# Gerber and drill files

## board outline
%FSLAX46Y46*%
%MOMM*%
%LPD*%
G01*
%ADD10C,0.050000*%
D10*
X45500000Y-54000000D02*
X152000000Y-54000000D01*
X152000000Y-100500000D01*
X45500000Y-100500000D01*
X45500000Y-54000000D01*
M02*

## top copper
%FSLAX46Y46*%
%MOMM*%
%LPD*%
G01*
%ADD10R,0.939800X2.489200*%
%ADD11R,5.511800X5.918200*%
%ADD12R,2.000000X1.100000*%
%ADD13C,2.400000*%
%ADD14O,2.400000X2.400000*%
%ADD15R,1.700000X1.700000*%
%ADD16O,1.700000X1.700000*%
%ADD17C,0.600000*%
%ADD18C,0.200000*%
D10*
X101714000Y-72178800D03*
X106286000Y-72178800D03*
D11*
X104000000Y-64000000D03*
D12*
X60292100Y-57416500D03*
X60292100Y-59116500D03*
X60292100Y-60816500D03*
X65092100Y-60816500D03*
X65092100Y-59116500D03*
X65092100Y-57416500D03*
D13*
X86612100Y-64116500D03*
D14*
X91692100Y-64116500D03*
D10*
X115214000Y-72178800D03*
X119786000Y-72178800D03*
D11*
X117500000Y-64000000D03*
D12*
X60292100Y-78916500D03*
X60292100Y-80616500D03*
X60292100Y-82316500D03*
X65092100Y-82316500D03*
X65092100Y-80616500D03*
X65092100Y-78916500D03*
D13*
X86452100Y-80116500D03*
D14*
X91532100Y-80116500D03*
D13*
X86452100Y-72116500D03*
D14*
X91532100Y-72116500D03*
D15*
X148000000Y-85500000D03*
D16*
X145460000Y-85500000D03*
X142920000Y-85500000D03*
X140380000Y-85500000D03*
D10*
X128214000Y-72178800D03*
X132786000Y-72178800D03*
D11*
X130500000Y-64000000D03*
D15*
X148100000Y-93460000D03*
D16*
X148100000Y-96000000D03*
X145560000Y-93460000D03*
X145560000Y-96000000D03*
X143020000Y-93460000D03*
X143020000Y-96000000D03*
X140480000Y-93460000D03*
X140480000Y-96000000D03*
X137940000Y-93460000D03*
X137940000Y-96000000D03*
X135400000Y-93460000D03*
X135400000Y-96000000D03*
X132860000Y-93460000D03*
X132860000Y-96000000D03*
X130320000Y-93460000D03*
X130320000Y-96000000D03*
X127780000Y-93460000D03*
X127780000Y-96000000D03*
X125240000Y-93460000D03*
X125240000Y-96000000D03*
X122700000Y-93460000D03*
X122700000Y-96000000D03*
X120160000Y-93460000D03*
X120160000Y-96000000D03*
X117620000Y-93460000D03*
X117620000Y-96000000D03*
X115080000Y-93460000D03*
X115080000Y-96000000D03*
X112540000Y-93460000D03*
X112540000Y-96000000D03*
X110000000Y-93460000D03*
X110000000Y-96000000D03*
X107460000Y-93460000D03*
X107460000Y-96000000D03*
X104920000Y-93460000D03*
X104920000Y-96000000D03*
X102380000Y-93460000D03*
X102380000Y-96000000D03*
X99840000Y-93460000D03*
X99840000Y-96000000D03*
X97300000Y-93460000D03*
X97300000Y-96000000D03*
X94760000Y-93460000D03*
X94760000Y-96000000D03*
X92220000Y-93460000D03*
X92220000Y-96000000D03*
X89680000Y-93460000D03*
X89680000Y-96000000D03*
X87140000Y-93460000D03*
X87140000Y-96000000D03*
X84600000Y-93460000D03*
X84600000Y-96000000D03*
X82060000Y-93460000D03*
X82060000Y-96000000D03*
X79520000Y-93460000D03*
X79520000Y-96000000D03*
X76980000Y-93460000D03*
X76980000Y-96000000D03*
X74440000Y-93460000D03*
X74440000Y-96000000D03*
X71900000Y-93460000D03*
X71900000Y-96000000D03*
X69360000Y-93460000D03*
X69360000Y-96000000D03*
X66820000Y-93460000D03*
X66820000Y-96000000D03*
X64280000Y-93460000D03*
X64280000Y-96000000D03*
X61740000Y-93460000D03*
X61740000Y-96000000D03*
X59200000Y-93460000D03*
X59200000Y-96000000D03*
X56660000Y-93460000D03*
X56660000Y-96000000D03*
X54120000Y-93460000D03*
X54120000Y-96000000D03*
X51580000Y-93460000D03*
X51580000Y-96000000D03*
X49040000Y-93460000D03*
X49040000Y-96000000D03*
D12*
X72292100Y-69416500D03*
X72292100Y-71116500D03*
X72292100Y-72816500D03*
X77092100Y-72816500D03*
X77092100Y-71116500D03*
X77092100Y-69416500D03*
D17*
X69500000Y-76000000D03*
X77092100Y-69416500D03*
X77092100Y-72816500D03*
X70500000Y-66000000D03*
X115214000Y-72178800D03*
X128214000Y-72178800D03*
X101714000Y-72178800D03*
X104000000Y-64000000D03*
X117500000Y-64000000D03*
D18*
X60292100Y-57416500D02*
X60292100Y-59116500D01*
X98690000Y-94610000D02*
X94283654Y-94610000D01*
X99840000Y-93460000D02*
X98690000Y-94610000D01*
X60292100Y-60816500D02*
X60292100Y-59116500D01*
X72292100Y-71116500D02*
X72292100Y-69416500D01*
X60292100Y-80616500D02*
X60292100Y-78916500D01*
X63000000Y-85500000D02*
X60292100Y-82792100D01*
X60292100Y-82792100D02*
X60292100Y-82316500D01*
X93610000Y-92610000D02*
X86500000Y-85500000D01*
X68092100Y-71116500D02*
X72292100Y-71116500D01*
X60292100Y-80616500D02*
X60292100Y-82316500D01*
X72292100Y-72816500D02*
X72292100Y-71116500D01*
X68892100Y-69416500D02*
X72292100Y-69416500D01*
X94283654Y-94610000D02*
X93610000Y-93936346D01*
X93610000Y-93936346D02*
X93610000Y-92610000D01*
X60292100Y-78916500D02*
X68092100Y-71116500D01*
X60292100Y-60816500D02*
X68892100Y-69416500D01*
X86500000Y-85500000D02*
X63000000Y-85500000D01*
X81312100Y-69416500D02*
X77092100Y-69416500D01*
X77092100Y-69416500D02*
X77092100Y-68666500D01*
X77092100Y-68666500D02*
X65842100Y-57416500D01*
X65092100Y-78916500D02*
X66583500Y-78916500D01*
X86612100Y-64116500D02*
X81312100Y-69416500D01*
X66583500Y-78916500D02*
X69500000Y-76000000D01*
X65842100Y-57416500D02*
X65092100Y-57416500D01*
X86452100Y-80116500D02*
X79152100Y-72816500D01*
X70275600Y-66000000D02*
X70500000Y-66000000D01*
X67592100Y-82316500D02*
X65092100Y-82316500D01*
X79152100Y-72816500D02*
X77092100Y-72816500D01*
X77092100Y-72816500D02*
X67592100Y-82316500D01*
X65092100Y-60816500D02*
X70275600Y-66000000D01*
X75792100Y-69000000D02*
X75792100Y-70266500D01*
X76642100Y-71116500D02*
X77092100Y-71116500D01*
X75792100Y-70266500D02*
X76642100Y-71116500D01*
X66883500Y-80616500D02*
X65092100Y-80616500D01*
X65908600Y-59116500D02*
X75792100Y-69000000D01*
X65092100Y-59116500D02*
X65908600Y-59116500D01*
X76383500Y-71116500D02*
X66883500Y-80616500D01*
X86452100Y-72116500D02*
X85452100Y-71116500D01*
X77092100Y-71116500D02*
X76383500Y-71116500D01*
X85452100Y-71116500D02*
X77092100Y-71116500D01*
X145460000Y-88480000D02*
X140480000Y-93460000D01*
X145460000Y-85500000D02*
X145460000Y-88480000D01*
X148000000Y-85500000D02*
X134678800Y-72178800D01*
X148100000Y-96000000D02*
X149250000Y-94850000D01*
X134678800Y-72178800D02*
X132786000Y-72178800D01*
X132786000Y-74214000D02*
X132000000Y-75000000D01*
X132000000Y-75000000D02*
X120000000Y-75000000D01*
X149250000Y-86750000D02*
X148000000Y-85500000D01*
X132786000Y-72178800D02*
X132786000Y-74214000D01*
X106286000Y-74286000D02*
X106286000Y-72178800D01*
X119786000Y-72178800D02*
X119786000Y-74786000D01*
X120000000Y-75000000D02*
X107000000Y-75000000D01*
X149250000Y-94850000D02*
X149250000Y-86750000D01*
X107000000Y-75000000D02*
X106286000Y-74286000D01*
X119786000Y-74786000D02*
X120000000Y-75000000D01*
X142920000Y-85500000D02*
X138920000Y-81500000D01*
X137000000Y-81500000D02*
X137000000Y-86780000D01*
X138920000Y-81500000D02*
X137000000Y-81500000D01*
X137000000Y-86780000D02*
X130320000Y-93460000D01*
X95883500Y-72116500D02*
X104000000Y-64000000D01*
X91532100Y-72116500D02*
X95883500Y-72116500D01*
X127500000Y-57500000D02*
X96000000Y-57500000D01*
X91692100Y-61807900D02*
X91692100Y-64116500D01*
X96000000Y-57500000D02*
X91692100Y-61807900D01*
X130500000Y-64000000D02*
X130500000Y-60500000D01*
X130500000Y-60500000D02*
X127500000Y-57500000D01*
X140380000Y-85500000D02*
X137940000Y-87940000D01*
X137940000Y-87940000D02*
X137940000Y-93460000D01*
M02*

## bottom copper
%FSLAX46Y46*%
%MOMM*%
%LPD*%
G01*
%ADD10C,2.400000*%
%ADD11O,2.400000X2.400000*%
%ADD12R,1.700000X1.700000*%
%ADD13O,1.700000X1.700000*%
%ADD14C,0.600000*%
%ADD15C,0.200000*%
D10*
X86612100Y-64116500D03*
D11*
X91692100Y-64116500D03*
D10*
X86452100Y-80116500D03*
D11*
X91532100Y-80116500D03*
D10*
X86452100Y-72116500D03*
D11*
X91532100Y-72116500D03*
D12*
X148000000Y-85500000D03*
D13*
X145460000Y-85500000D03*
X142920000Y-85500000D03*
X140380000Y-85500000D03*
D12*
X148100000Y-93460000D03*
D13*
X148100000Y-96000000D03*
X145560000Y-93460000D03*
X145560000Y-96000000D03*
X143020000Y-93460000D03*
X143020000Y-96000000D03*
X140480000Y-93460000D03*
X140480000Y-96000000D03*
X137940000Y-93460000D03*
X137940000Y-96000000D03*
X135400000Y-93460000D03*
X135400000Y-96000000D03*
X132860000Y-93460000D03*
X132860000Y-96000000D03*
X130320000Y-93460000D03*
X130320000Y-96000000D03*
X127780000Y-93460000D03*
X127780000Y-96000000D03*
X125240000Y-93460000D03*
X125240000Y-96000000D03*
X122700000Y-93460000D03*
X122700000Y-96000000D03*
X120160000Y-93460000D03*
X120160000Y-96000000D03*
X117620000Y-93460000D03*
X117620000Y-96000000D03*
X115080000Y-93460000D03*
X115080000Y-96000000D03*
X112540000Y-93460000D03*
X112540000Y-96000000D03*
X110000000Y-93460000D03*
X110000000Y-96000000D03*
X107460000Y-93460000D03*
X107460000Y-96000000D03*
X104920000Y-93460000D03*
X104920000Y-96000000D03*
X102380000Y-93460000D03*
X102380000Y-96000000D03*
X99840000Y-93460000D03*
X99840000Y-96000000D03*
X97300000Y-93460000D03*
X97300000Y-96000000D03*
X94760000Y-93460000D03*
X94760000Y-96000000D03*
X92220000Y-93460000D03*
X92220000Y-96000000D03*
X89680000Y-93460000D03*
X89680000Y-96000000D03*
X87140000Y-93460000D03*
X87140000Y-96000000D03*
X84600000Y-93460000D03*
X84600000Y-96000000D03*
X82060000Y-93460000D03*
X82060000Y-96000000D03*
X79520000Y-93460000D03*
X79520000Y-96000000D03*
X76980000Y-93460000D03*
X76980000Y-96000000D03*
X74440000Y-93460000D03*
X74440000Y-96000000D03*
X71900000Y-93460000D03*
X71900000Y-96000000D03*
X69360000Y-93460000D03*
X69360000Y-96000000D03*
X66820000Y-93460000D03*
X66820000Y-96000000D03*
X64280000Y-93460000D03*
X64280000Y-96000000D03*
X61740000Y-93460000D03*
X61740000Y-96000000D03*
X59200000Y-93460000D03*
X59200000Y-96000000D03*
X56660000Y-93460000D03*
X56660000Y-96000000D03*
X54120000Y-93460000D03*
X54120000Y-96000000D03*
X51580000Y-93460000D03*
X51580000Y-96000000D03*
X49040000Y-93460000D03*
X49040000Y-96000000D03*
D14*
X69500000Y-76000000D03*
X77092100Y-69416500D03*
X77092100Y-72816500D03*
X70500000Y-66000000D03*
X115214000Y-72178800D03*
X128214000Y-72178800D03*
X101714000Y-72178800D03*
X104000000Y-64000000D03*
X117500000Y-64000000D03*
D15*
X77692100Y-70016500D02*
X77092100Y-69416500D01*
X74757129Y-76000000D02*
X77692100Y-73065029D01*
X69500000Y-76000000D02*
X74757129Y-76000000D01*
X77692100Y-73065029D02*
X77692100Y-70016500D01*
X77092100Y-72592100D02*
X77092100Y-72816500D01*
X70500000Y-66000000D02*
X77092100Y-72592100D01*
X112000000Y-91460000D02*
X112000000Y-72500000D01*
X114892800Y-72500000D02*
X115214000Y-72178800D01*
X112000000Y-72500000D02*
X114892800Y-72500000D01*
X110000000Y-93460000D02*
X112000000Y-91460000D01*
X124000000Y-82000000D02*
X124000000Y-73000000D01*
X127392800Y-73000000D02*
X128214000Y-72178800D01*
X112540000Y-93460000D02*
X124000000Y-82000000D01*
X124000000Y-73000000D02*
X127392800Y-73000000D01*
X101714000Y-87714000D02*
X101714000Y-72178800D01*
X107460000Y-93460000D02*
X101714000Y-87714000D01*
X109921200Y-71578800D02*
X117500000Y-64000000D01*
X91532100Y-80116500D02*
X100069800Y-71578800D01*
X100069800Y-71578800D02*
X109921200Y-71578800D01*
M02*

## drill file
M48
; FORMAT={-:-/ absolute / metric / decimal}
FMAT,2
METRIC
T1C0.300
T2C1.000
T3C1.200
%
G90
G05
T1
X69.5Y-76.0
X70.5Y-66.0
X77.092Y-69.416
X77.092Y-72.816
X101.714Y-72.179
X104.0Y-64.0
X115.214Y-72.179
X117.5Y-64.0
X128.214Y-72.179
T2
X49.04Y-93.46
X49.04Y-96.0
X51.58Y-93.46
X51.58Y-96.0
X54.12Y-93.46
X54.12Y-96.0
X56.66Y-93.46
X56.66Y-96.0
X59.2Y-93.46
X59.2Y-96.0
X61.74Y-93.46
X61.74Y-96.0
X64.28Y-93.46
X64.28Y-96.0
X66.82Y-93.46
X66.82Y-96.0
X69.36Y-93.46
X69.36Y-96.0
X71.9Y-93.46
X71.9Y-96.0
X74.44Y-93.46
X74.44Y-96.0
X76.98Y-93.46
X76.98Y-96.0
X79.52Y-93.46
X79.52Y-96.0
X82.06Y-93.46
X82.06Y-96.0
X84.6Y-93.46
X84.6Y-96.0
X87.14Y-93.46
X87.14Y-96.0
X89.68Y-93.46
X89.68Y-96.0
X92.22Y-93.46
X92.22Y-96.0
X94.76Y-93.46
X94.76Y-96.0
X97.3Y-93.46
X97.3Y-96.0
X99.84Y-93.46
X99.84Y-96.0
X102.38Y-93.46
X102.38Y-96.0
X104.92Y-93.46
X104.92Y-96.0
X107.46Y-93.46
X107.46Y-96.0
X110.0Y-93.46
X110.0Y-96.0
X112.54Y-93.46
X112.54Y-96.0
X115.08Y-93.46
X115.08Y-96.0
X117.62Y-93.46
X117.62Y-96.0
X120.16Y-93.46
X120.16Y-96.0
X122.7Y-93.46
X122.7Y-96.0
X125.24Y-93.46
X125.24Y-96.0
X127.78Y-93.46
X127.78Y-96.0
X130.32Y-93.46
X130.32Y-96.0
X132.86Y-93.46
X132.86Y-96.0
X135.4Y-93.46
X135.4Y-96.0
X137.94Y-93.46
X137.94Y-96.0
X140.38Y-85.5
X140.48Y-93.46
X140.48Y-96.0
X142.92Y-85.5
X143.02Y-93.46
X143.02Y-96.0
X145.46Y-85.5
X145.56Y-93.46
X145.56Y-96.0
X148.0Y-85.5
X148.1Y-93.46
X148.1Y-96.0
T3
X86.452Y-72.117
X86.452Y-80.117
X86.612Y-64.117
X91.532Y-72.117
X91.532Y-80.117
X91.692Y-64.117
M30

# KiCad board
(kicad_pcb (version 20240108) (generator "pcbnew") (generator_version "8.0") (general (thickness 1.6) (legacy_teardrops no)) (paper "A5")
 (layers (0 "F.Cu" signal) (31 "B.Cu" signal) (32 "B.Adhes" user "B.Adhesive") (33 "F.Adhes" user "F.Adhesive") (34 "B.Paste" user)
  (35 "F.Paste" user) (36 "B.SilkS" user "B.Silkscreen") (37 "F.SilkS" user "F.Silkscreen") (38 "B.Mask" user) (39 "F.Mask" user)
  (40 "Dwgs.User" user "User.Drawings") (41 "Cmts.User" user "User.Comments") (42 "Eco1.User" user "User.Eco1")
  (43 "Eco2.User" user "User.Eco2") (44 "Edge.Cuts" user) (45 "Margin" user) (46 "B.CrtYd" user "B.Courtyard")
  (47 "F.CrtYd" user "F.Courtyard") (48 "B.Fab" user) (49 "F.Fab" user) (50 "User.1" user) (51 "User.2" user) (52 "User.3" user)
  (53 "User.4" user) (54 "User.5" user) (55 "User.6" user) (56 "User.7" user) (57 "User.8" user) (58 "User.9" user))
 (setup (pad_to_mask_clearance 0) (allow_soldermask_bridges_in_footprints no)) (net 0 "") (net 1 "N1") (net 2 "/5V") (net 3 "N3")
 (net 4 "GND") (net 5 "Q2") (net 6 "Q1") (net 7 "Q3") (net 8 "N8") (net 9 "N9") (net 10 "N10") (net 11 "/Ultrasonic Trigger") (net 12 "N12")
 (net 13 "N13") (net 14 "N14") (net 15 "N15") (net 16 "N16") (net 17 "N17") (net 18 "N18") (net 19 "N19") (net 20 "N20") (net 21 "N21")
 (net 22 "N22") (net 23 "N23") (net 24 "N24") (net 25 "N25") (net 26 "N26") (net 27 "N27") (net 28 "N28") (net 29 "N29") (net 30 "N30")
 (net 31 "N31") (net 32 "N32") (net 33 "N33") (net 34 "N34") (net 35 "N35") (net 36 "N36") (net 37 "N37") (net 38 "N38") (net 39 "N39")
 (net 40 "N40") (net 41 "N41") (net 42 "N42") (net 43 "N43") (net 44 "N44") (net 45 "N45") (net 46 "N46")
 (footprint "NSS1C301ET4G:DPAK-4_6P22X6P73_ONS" (layer "F.Cu") (at 104 65.7653)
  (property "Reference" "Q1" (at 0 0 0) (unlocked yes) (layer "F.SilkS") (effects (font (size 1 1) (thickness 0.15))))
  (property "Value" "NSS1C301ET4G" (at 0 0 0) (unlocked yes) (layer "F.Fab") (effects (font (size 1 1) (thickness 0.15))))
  (pad "1" smd rect (at -2.286 6.4135) (size 0.9398 2.4892) (layers "F.Cu" "F.Paste" "F.Mask") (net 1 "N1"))
  (pad "2" smd rect (at 2.286 6.4135) (size 0.9398 2.4892) (layers "F.Cu" "F.Paste" "F.Mask") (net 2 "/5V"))
  (pad "3" smd rect (at 0 -1.7653) (size 5.5118 5.9182) (layers "F.Cu" "F.Paste" "F.Mask") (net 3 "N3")))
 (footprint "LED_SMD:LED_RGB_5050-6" (layer "F.Cu") (at 62.6921 59.1165)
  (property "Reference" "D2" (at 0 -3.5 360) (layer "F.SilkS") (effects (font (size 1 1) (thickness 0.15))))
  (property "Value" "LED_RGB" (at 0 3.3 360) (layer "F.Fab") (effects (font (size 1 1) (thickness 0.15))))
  (pad "1" smd rect (at -2.4 -1.7 90) (size 1.1 2) (layers "F.Cu" "F.Paste" "F.Mask") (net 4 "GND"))
  (pad "2" smd rect (at -2.4 0 90) (size 1.1 2) (layers "F.Cu" "F.Paste" "F.Mask") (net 4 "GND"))
  (pad "3" smd rect (at -2.4 1.7 90) (size 1.1 2) (layers "F.Cu" "F.Paste" "F.Mask") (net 4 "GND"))
  (pad "4" smd rect (at 2.4 1.7 90) (size 1.1 2) (layers "F.Cu" "F.Paste" "F.Mask") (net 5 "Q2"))
  (pad "5" smd rect (at 2.4 0 90) (size 1.1 2) (layers "F.Cu" "F.Paste" "F.Mask") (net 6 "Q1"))
  (pad "6" smd rect (at 2.4 -1.7 90) (size 1.1 2) (layers "F.Cu" "F.Paste" "F.Mask") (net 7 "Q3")))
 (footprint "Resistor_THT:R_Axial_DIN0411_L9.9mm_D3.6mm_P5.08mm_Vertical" (layer "F.Cu") (at 86.6121 64.1165)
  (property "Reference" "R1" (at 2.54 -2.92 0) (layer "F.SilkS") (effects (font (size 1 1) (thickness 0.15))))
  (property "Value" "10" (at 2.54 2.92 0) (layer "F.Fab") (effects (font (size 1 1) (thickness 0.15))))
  (pad "1" thru_hole circle (at 0 0) (size 2.4 2.4) (drill 1.2) (layers "*.Cu" "*.Mask") (remove_unused_layers no) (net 7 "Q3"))
  (pad "2" thru_hole oval (at 5.08 0) (size 2.4 2.4) (drill 1.2) (layers "*.Cu" "*.Mask") (remove_unused_layers no) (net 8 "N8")))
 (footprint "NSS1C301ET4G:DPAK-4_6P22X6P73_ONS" (layer "F.Cu") (at 117.5 65.7653)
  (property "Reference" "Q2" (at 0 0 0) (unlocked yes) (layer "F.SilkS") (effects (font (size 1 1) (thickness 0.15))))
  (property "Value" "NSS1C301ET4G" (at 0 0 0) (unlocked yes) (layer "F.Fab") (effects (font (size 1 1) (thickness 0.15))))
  (pad "1" smd rect (at -2.286 6.4135) (size 0.9398 2.4892) (layers "F.Cu" "F.Paste" "F.Mask") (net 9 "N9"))
  (pad "2" smd rect (at 2.286 6.4135) (size 0.9398 2.4892) (layers "F.Cu" "F.Paste" "F.Mask") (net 2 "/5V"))
  (pad "3" smd rect (at 0 -1.7653) (size 5.5118 5.9182) (layers "F.Cu" "F.Paste" "F.Mask") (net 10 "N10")))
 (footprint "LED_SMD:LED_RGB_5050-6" (layer "F.Cu") (at 62.6921 80.6165)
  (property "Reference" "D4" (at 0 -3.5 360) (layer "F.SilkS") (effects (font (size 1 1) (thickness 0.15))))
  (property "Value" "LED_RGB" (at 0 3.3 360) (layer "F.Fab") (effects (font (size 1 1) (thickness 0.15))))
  (pad "1" smd rect (at -2.4 -1.7 90) (size 1.1 2) (layers "F.Cu" "F.Paste" "F.Mask") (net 4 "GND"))
  (pad "2" smd rect (at -2.4 0 90) (size 1.1 2) (layers "F.Cu" "F.Paste" "F.Mask") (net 4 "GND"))
  (pad "3" smd rect (at -2.4 1.7 90) (size 1.1 2) (layers "F.Cu" "F.Paste" "F.Mask") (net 4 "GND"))
  (pad "4" smd rect (at 2.4 1.7 90) (size 1.1 2) (layers "F.Cu" "F.Paste" "F.Mask") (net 5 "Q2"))
  (pad "5" smd rect (at 2.4 0 90) (size 1.1 2) (layers "F.Cu" "F.Paste" "F.Mask") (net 6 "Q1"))
  (pad "6" smd rect (at 2.4 -1.7 90) (size 1.1 2) (layers "F.Cu" "F.Paste" "F.Mask") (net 7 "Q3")))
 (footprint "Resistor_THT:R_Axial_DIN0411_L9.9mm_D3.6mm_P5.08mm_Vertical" (layer "F.Cu") (at 86.4521 80.1165)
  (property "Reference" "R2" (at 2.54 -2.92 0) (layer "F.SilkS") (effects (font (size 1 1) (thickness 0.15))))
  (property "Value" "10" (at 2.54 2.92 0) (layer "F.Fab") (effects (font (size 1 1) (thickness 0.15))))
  (pad "1" thru_hole circle (at 0 0) (size 2.4 2.4) (drill 1.2) (layers "*.Cu" "*.Mask") (remove_unused_layers no) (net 5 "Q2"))
  (pad "2" thru_hole oval (at 5.08 0) (size 2.4 2.4) (drill 1.2) (layers "*.Cu" "*.Mask") (remove_unused_layers no) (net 10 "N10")))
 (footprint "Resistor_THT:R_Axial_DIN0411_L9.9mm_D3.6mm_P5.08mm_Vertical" (layer "F.Cu") (at 86.4521 72.1165)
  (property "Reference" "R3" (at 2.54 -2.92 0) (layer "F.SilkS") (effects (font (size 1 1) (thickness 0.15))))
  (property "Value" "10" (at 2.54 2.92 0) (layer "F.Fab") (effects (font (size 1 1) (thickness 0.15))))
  (pad "1" thru_hole circle (at 0 0) (size 2.4 2.4) (drill 1.2) (layers "*.Cu" "*.Mask") (remove_unused_layers no) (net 6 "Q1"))
  (pad "2" thru_hole oval (at 5.08 0) (size 2.4 2.4) (drill 1.2) (layers "*.Cu" "*.Mask") (remove_unused_layers no) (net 3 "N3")))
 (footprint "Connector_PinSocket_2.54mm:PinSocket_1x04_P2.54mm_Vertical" (layer "F.Cu") (at 148 85.5 -90)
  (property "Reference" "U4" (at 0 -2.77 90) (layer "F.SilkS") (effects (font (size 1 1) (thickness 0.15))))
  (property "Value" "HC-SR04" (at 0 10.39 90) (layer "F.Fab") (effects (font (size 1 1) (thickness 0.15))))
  (pad "1" thru_hole rect (at 0 0 270) (size 1.7 1.7) (drill 1) (layers "*.Cu" "*.Mask") (remove_unused_layers no) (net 2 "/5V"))
  (pad "2" thru_hole oval (at 0 2.54 270) (size 1.7 1.7) (drill 1) (layers "*.Cu" "*.Mask") (remove_unused_layers no)
   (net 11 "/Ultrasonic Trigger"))
  (pad "3" thru_hole oval (at 0 5.08 270) (size 1.7 1.7) (drill 1) (layers "*.Cu" "*.Mask") (remove_unused_layers no) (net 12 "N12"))
  (pad "4" thru_hole oval (at 0 7.62 270) (size 1.7 1.7) (drill 1) (layers "*.Cu" "*.Mask") (remove_unused_layers no) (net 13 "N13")))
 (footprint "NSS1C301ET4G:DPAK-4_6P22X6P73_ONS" (layer "F.Cu") (at 130.5 65.7653)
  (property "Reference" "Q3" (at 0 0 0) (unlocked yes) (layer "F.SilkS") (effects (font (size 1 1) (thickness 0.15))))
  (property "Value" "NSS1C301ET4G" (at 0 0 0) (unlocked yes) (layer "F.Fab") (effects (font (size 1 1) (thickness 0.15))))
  (pad "1" smd rect (at -2.286 6.4135) (size 0.9398 2.4892) (layers "F.Cu" "F.Paste" "F.Mask") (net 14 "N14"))
  (pad "2" smd rect (at 2.286 6.4135) (size 0.9398 2.4892) (layers "F.Cu" "F.Paste" "F.Mask") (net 2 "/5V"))
  (pad "3" smd rect (at 0 -1.7653) (size 5.5118 5.9182) (layers "F.Cu" "F.Paste" "F.Mask") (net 8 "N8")))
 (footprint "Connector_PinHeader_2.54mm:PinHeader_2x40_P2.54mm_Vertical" (layer "F.Cu") (at 148.1 93.46 -90)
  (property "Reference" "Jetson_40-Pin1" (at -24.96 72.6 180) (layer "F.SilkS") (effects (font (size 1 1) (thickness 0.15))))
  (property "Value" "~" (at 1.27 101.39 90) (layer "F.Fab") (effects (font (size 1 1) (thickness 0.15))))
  (pad "1" thru_hole rect (at 0 0 270) (size 1.7 1.7) (drill 1) (layers "*.Cu" "*.Mask") (remove_unused_layers no) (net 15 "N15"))
  (pad "2" thru_hole oval (at 2.54 0 270) (size 1.7 1.7) (drill 1) (layers "*.Cu" "*.Mask") (remove_unused_layers no) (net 2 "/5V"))
  (pad "3" thru_hole oval (at 0 2.54 270) (size 1.7 1.7) (drill 1) (layers "*.Cu" "*.Mask") (remove_unused_layers no) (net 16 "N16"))
  (pad "4" thru_hole oval (at 2.54 2.54 270) (size 1.7 1.7) (drill 1) (layers "*.Cu" "*.Mask") (remove_unused_layers no) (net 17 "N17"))
  (pad "5" thru_hole oval (at 0 5.08 270) (size 1.7 1.7) (drill 1) (layers "*.Cu" "*.Mask") (remove_unused_layers no) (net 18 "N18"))
  (pad "6" thru_hole oval (at 2.54 5.08 270) (size 1.7 1.7) (drill 1) (layers "*.Cu" "*.Mask") (remove_unused_layers no) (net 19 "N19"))
  (pad "7" thru_hole oval (at 0 7.62 270) (size 1.7 1.7) (drill 1) (layers "*.Cu" "*.Mask") (remove_unused_layers no)
   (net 11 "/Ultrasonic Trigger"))
  (pad "8" thru_hole oval (at 2.54 7.62 270) (size 1.7 1.7) (drill 1) (layers "*.Cu" "*.Mask") (remove_unused_layers no) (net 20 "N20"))
  (pad "9" thru_hole oval (at 0 10.16 270) (size 1.7 1.7) (drill 1) (layers "*.Cu" "*.Mask") (remove_unused_layers no) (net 13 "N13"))
  (pad "10" thru_hole oval (at 2.54 10.16 270) (size 1.7 1.7) (drill 1) (layers "*.Cu" "*.Mask") (remove_unused_layers no) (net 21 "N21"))
  (pad "11" thru_hole oval (at 0 12.7 270) (size 1.7 1.7) (drill 1) (layers "*.Cu" "*.Mask") (remove_unused_layers no) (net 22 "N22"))
  (pad "12" thru_hole oval (at 2.54 12.7 270) (size 1.7 1.7) (drill 1) (layers "*.Cu" "*.Mask") (remove_unused_layers no) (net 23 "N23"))
  (pad "13" thru_hole oval (at 0 15.24 270) (size 1.7 1.7) (drill 1) (layers "*.Cu" "*.Mask") (remove_unused_layers no) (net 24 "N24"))
  (pad "14" thru_hole oval (at 2.54 15.24 270) (size 1.7 1.7) (drill 1) (layers "*.Cu" "*.Mask") (remove_unused_layers no) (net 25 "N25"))
  (pad "15" thru_hole oval (at 0 17.78 270) (size 1.7 1.7) (drill 1) (layers "*.Cu" "*.Mask") (remove_unused_layers no) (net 12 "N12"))
  (pad "16" thru_hole oval (at 2.54 17.78 270) (size 1.7 1.7) (drill 1) (layers "*.Cu" "*.Mask") (remove_unused_layers no) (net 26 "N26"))
  (pad "17" thru_hole oval (at 0 20.32 270) (size 1.7 1.7) (drill 1) (layers "*.Cu" "*.Mask") (remove_unused_layers no) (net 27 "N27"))
  (pad "18" thru_hole oval (at 2.54 20.32 270) (size 1.7 1.7) (drill 1) (layers "*.Cu" "*.Mask") (remove_unused_layers no) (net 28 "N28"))
  (pad "19" thru_hole oval (at 0 22.86 270) (size 1.7 1.7) (drill 1) (layers "*.Cu" "*.Mask") (remove_unused_layers no) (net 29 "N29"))
  (pad "20" thru_hole oval (at 2.54 22.86 270) (size 1.7 1.7) (drill 1) (layers "*.Cu" "*.Mask") (remove_unused_layers no) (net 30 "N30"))
  (pad "21" thru_hole oval (at 0 25.4 270) (size 1.7 1.7) (drill 1) (layers "*.Cu" "*.Mask") (remove_unused_layers no) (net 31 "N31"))
  (pad "22" thru_hole oval (at 2.54 25.4 270) (size 1.7 1.7) (drill 1) (layers "*.Cu" "*.Mask") (remove_unused_layers no) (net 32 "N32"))
  (pad "23" thru_hole oval (at 0 27.94 270) (size 1.7 1.7) (drill 1) (layers "*.Cu" "*.Mask") (remove_unused_layers no) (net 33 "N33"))
  (pad "24" thru_hole oval (at 2.54 27.94 270) (size 1.7 1.7) (drill 1) (layers "*.Cu" "*.Mask") (remove_unused_layers no) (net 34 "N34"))
  (pad "25" thru_hole oval (at 0 30.48 270) (size 1.7 1.7) (drill 1) (layers "*.Cu" "*.Mask") (remove_unused_layers no) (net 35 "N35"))
  (pad "26" thru_hole oval (at 2.54 30.48 270) (size 1.7 1.7) (drill 1) (layers "*.Cu" "*.Mask") (remove_unused_layers no) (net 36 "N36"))
  (pad "27" thru_hole oval (at 0 33.02 270) (size 1.7 1.7) (drill 1) (layers "*.Cu" "*.Mask") (remove_unused_layers no) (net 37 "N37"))
  (pad "28" thru_hole oval (at 2.54 33.02 270) (size 1.7 1.7) (drill 1) (layers "*.Cu" "*.Mask") (remove_unused_layers no) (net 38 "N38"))
  (pad "29" thru_hole oval (at 0 35.56 270) (size 1.7 1.7) (drill 1) (layers "*.Cu" "*.Mask") (remove_unused_layers no) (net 14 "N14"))
  (pad "30" thru_hole oval (at 2.54 35.56 270) (size 1.7 1.7) (drill 1) (layers "*.Cu" "*.Mask") (remove_unused_layers no) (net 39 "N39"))
  (pad "31" thru_hole oval (at 0 38.1 270) (size 1.7 1.7) (drill 1) (layers "*.Cu" "*.Mask") (remove_unused_layers no) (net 9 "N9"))
  (pad "32" thru_hole oval (at 2.54 38.1 270) (size 1.7 1.7) (drill 1) (layers "*.Cu" "*.Mask") (remove_unused_layers no) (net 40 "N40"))
  (pad "33" thru_hole oval (at 0 40.64 270) (size 1.7 1.7) (drill 1) (layers "*.Cu" "*.Mask") (remove_unused_layers no) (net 1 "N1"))
  (pad "34" thru_hole oval (at 2.54 40.64 270) (size 1.7 1.7) (drill 1) (layers "*.Cu" "*.Mask") (remove_unused_layers no) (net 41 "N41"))
  (pad "35" thru_hole oval (at 0 43.18 270) (size 1.7 1.7) (drill 1) (layers "*.Cu" "*.Mask") (remove_unused_layers no) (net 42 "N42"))
  (pad "36" thru_hole oval (at 2.54 43.18 270) (size 1.7 1.7) (drill 1) (layers "*.Cu" "*.Mask") (remove_unused_layers no) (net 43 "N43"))
  (pad "37" thru_hole oval (at 0 45.72 270) (size 1.7 1.7) (drill 1) (layers "*.Cu" "*.Mask") (remove_unused_layers no) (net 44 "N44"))
  (pad "38" thru_hole oval (at 2.54 45.72 270) (size 1.7 1.7) (drill 1) (layers "*.Cu" "*.Mask") (remove_unused_layers no) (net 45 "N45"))
  (pad "39" thru_hole oval (at 0 48.26 270) (size 1.7 1.7) (drill 1) (layers "*.Cu" "*.Mask") (remove_unused_layers no) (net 4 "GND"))
  (pad "40" thru_hole oval (at 2.54 48.26 270) (size 1.7 1.7) (drill 1) (layers "*.Cu" "*.Mask") (remove_unused_layers no) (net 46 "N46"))
  (pad "41" thru_hole oval (at 0 50.8 270) (size 1.7 1.7) (drill 1) (layers "*.Cu" "*.Mask") (remove_unused_layers no))
  (pad "42" thru_hole oval (at 2.54 50.8 270) (size 1.7 1.7) (drill 1) (layers "*.Cu" "*.Mask") (remove_unused_layers no))
  (pad "43" thru_hole oval (at 0 53.34 270) (size 1.7 1.7) (drill 1) (layers "*.Cu" "*.Mask") (remove_unused_layers no))
  (pad "44" thru_hole oval (at 2.54 53.34 270) (size 1.7 1.7) (drill 1) (layers "*.Cu" "*.Mask") (remove_unused_layers no))
  (pad "45" thru_hole oval (at 0 55.88 270) (size 1.7 1.7) (drill 1) (layers "*.Cu" "*.Mask") (remove_unused_layers no))
  (pad "46" thru_hole oval (at 2.54 55.88 270) (size 1.7 1.7) (drill 1) (layers "*.Cu" "*.Mask") (remove_unused_layers no))
  (pad "47" thru_hole oval (at 0 58.42 270) (size 1.7 1.7) (drill 1) (layers "*.Cu" "*.Mask") (remove_unused_layers no))
  (pad "48" thru_hole oval (at 2.54 58.42 270) (size 1.7 1.7) (drill 1) (layers "*.Cu" "*.Mask") (remove_unused_layers no))
  (pad "49" thru_hole oval (at 0 60.96 270) (size 1.7 1.7) (drill 1) (layers "*.Cu" "*.Mask") (remove_unused_layers no))
  (pad "50" thru_hole oval (at 2.54 60.96 270) (size 1.7 1.7) (drill 1) (layers "*.Cu" "*.Mask") (remove_unused_layers no))
  (pad "51" thru_hole oval (at 0 63.5 270) (size 1.7 1.7) (drill 1) (layers "*.Cu" "*.Mask") (remove_unused_layers no))
  (pad "52" thru_hole oval (at 2.54 63.5 270) (size 1.7 1.7) (drill 1) (layers "*.Cu" "*.Mask") (remove_unused_layers no))
  (pad "53" thru_hole oval (at 0 66.04 270) (size 1.7 1.7) (drill 1) (layers "*.Cu" "*.Mask") (remove_unused_layers no))
  (pad "54" thru_hole oval (at 2.54 66.04 270) (size 1.7 1.7) (drill 1) (layers "*.Cu" "*.Mask") (remove_unused_layers no))
  (pad "55" thru_hole oval (at 0 68.58 270) (size 1.7 1.7) (drill 1) (layers "*.Cu" "*.Mask") (remove_unused_layers no))
  (pad "56" thru_hole oval (at 2.54 68.58 270) (size 1.7 1.7) (drill 1) (layers "*.Cu" "*.Mask") (remove_unused_layers no))
  (pad "57" thru_hole oval (at 0 71.12 270) (size 1.7 1.7) (drill 1) (layers "*.Cu" "*.Mask") (remove_unused_layers no))
  (pad "58" thru_hole oval (at 2.54 71.12 270) (size 1.7 1.7) (drill 1) (layers "*.Cu" "*.Mask") (remove_unused_layers no))
  (pad "59" thru_hole oval (at 0 73.66 270) (size 1.7 1.7) (drill 1) (layers "*.Cu" "*.Mask") (remove_unused_layers no))
  (pad "60" thru_hole oval (at 2.54 73.66 270) (size 1.7 1.7) (drill 1) (layers "*.Cu" "*.Mask") (remove_unused_layers no))
  (pad "61" thru_hole oval (at 0 76.2 270) (size 1.7 1.7) (drill 1) (layers "*.Cu" "*.Mask") (remove_unused_layers no))
  (pad "62" thru_hole oval (at 2.54 76.2 270) (size 1.7 1.7) (drill 1) (layers "*.Cu" "*.Mask") (remove_unused_layers no))
  (pad "63" thru_hole oval (at 0 78.74 270) (size 1.7 1.7) (drill 1) (layers "*.Cu" "*.Mask") (remove_unused_layers no))
  (pad "64" thru_hole oval (at 2.54 78.74 270) (size 1.7 1.7) (drill 1) (layers "*.Cu" "*.Mask") (remove_unused_layers no))
  (pad "65" thru_hole oval (at 0 81.28 270) (size 1.7 1.7) (drill 1) (layers "*.Cu" "*.Mask") (remove_unused_layers no))
  (pad "66" thru_hole oval (at 2.54 81.28 270) (size 1.7 1.7) (drill 1) (layers "*.Cu" "*.Mask") (remove_unused_layers no))
  (pad "67" thru_hole oval (at 0 83.82 270) (size 1.7 1.7) (drill 1) (layers "*.Cu" "*.Mask") (remove_unused_layers no))
  (pad "68" thru_hole oval (at 2.54 83.82 270) (size 1.7 1.7) (drill 1) (layers "*.Cu" "*.Mask") (remove_unused_layers no))
  (pad "69" thru_hole oval (at 0 86.36 270) (size 1.7 1.7) (drill 1) (layers "*.Cu" "*.Mask") (remove_unused_layers no))
  (pad "70" thru_hole oval (at 2.54 86.36 270) (size 1.7 1.7) (drill 1) (layers "*.Cu" "*.Mask") (remove_unused_layers no))
  (pad "71" thru_hole oval (at 0 88.9 270) (size 1.7 1.7) (drill 1) (layers "*.Cu" "*.Mask") (remove_unused_layers no))
  (pad "72" thru_hole oval (at 2.54 88.9 270) (size 1.7 1.7) (drill 1) (layers "*.Cu" "*.Mask") (remove_unused_layers no))
  (pad "73" thru_hole oval (at 0 91.44 270) (size 1.7 1.7) (drill 1) (layers "*.Cu" "*.Mask") (remove_unused_layers no))
  (pad "74" thru_hole oval (at 2.54 91.44 270) (size 1.7 1.7) (drill 1) (layers "*.Cu" "*.Mask") (remove_unused_layers no))
  (pad "75" thru_hole oval (at 0 93.98 270) (size 1.7 1.7) (drill 1) (layers "*.Cu" "*.Mask") (remove_unused_layers no))
  (pad "76" thru_hole oval (at 2.54 93.98 270) (size 1.7 1.7) (drill 1) (layers "*.Cu" "*.Mask") (remove_unused_layers no))
  (pad "77" thru_hole oval (at 0 96.52 270) (size 1.7 1.7) (drill 1) (layers "*.Cu" "*.Mask") (remove_unused_layers no))
  (pad "78" thru_hole oval (at 2.54 96.52 270) (size 1.7 1.7) (drill 1) (layers "*.Cu" "*.Mask") (remove_unused_layers no))
  (pad "79" thru_hole oval (at 0 99.06 270) (size 1.7 1.7) (drill 1) (layers "*.Cu" "*.Mask") (remove_unused_layers no))
  (pad "80" thru_hole oval (at 2.54 99.06 270) (size 1.7 1.7) (drill 1) (layers "*.Cu" "*.Mask") (remove_unused_layers no)))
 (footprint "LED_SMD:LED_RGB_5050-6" (layer "F.Cu") (at 74.6921 71.1165)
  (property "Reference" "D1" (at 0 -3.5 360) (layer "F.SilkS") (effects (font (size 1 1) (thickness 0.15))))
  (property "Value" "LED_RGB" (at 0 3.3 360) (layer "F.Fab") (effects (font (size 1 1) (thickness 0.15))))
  (pad "1" smd rect (at -2.4 -1.7 90) (size 1.1 2) (layers "F.Cu" "F.Paste" "F.Mask") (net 4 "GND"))
  (pad "2" smd rect (at -2.4 0 90) (size 1.1 2) (layers "F.Cu" "F.Paste" "F.Mask") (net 4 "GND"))
  (pad "3" smd rect (at -2.4 1.7 90) (size 1.1 2) (layers "F.Cu" "F.Paste" "F.Mask") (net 4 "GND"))
  (pad "4" smd rect (at 2.4 1.7 90) (size 1.1 2) (layers "F.Cu" "F.Paste" "F.Mask") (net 5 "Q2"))
  (pad "5" smd rect (at 2.4 0 90) (size 1.1 2) (layers "F.Cu" "F.Paste" "F.Mask") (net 6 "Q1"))
  (pad "6" smd rect (at 2.4 -1.7 90) (size 1.1 2) (layers "F.Cu" "F.Paste" "F.Mask") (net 7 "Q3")))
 (gr_rect (start 45.5 54) (end 152 100.5) (stroke (width 0.05) (type default)) (fill none) (layer "Edge.Cuts"))
 (segment (start 60.2921 57.4165) (end 60.2921 59.1165) (width 0.2) (layer "F.Cu") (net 4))
 (segment (start 98.69 94.61) (end 94.283654 94.61) (width 0.2) (layer "F.Cu") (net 4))
 (segment (start 99.84 93.46) (end 98.69 94.61) (width 0.2) (layer "F.Cu") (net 4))
 (segment (start 60.2921 60.8165) (end 60.2921 59.1165) (width 0.2) (layer "F.Cu") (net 4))
 (segment (start 72.2921 71.1165) (end 72.2921 69.4165) (width 0.2) (layer "F.Cu") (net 4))
 (segment (start 60.2921 80.6165) (end 60.2921 78.9165) (width 0.2) (layer "F.Cu") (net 4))
 (segment (start 63 85.5) (end 60.2921 82.7921) (width 0.2) (layer "F.Cu") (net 4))
 (segment (start 60.2921 82.7921) (end 60.2921 82.3165) (width 0.2) (layer "F.Cu") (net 4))
 (segment (start 93.61 92.61) (end 86.5 85.5) (width 0.2) (layer "F.Cu") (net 4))
 (segment (start 68.0921 71.1165) (end 72.2921 71.1165) (width 0.2) (layer "F.Cu") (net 4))
 (segment (start 60.2921 80.6165) (end 60.2921 82.3165) (width 0.2) (layer "F.Cu") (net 4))
 (segment (start 72.2921 72.8165) (end 72.2921 71.1165) (width 0.2) (layer "F.Cu") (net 4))
 (segment (start 68.8921 69.4165) (end 72.2921 69.4165) (width 0.2) (layer "F.Cu") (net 4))
 (segment (start 94.283654 94.61) (end 93.61 93.936346) (width 0.2) (layer "F.Cu") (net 4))
 (segment (start 93.61 93.936346) (end 93.61 92.61) (width 0.2) (layer "F.Cu") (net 4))
 (segment (start 60.2921 78.9165) (end 68.0921 71.1165) (width 0.2) (layer "F.Cu") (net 4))
 (segment (start 60.2921 60.8165) (end 68.8921 69.4165) (width 0.2) (layer "F.Cu") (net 4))
 (segment (start 86.5 85.5) (end 63 85.5) (width 0.2) (layer "F.Cu") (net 4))
 (segment (start 81.3121 69.4165) (end 77.0921 69.4165) (width 0.2) (layer "F.Cu") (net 7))
 (segment (start 77.0921 69.4165) (end 77.0921 68.6665) (width 0.2) (layer "F.Cu") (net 7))
 (segment (start 77.0921 68.6665) (end 65.8421 57.4165) (width 0.2) (layer "F.Cu") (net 7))
 (segment (start 65.0921 78.9165) (end 66.5835 78.9165) (width 0.2) (layer "F.Cu") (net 7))
 (segment (start 86.6121 64.1165) (end 81.3121 69.4165) (width 0.2) (layer "F.Cu") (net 7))
 (segment (start 66.5835 78.9165) (end 69.5 76) (width 0.2) (layer "F.Cu") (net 7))
 (segment (start 65.8421 57.4165) (end 65.0921 57.4165) (width 0.2) (layer "F.Cu") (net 7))
 (via (at 69.5 76) (size 0.6) (drill 0.3) (layers "F.Cu" "B.Cu") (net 7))
 (via (at 77.0921 69.4165) (size 0.6) (drill 0.3) (layers "F.Cu" "B.Cu") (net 7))
 (segment (start 77.6921 70.0165) (end 77.0921 69.4165) (width 0.2) (layer "B.Cu") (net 7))
 (segment (start 74.757129 76) (end 77.6921 73.065029) (width 0.2) (layer "B.Cu") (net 7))
 (segment (start 69.5 76) (end 74.757129 76) (width 0.2) (layer "B.Cu") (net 7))
 (segment (start 77.6921 73.065029) (end 77.6921 70.0165) (width 0.2) (layer "B.Cu") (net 7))
 (segment (start 86.4521 80.1165) (end 79.1521 72.8165) (width 0.2) (layer "F.Cu") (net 5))
 (segment (start 70.2756 66) (end 70.5 66) (width 0.2) (layer "F.Cu") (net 5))
 (segment (start 67.5921 82.3165) (end 65.0921 82.3165) (width 0.2) (layer "F.Cu") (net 5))
 (segment (start 79.1521 72.8165) (end 77.0921 72.8165) (width 0.2) (layer "F.Cu") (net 5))
 (segment (start 77.0921 72.8165) (end 67.5921 82.3165) (width 0.2) (layer "F.Cu") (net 5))
 (segment (start 65.0921 60.8165) (end 70.2756 66) (width 0.2) (layer "F.Cu") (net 5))
 (via (at 77.0921 72.8165) (size 0.6) (drill 0.3) (layers "F.Cu" "B.Cu") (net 5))
 (via (at 70.5 66) (size 0.6) (drill 0.3) (layers "F.Cu" "B.Cu") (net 5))
 (segment (start 77.0921 72.5921) (end 77.0921 72.8165) (width 0.2) (layer "B.Cu") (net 5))
 (segment (start 70.5 66) (end 77.0921 72.5921) (width 0.2) (layer "B.Cu") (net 5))
 (segment (start 75.7921 69) (end 75.7921 70.2665) (width 0.2) (layer "F.Cu") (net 6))
 (segment (start 76.6421 71.1165) (end 77.0921 71.1165) (width 0.2) (layer "F.Cu") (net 6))
 (segment (start 75.7921 70.2665) (end 76.6421 71.1165) (width 0.2) (layer "F.Cu") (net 6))
 (segment (start 66.8835 80.6165) (end 65.0921 80.6165) (width 0.2) (layer "F.Cu") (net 6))
 (segment (start 65.9086 59.1165) (end 75.7921 69) (width 0.2) (layer "F.Cu") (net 6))
 (segment (start 65.0921 59.1165) (end 65.9086 59.1165) (width 0.2) (layer "F.Cu") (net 6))
 (segment (start 76.3835 71.1165) (end 66.8835 80.6165) (width 0.2) (layer "F.Cu") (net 6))
 (segment (start 86.4521 72.1165) (end 85.4521 71.1165) (width 0.2) (layer "F.Cu") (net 6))
 (segment (start 77.0921 71.1165) (end 76.3835 71.1165) (width 0.2) (layer "F.Cu") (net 6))
 (segment (start 85.4521 71.1165) (end 77.0921 71.1165) (width 0.2) (layer "F.Cu") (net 6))
 (via (at 115.214 72.1788) (size 0.6) (drill 0.3) (layers "F.Cu" "B.Cu") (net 9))
 (segment (start 112 91.46) (end 112 72.5) (width 0.2) (layer "B.Cu") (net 9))
 (segment (start 114.8928 72.5) (end 115.214 72.1788) (width 0.2) (layer "B.Cu") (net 9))
 (segment (start 112 72.5) (end 114.8928 72.5) (width 0.2) (layer "B.Cu") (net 9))
 (segment (start 110 93.46) (end 112 91.46) (width 0.2) (layer "B.Cu") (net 9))
 (via (at 128.214 72.1788) (size 0.6) (drill 0.3) (layers "F.Cu" "B.Cu") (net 14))
 (segment (start 124 82) (end 124 73) (width 0.2) (layer "B.Cu") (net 14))
 (segment (start 127.3928 73) (end 128.214 72.1788) (width 0.2) (layer "B.Cu") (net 14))
 (segment (start 112.54 93.46) (end 124 82) (width 0.2) (layer "B.Cu") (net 14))
 (segment (start 124 73) (end 127.3928 73) (width 0.2) (layer "B.Cu") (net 14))
 (segment (start 145.46 88.48) (end 140.48 93.46) (width 0.2) (layer "F.Cu") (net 11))
 (segment (start 145.46 85.5) (end 145.46 88.48) (width 0.2) (layer "F.Cu") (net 11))
 (segment (start 148 85.5) (end 134.6788 72.1788) (width 0.2) (layer "F.Cu") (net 2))
 (segment (start 148.1 96) (end 149.25 94.85) (width 0.2) (layer "F.Cu") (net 2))
 (segment (start 134.6788 72.1788) (end 132.786 72.1788) (width 0.2) (layer "F.Cu") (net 2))
 (segment (start 132.786 74.214) (end 132 75) (width 0.2) (layer "F.Cu") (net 2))
 (segment (start 132 75) (end 120 75) (width 0.2) (layer "F.Cu") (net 2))
 (segment (start 149.25 86.75) (end 148 85.5) (width 0.2) (layer "F.Cu") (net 2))
 (segment (start 132.786 72.1788) (end 132.786 74.214) (width 0.2) (layer "F.Cu") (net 2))
 (segment (start 106.286 74.286) (end 106.286 72.1788) (width 0.2) (layer "F.Cu") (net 2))
 (segment (start 119.786 72.1788) (end 119.786 74.786) (width 0.2) (layer "F.Cu") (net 2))
 (segment (start 120 75) (end 107 75) (width 0.2) (layer "F.Cu") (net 2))
 (segment (start 149.25 94.85) (end 149.25 86.75) (width 0.2) (layer "F.Cu") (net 2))
 (segment (start 107 75) (end 106.286 74.286) (width 0.2) (layer "F.Cu") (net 2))
 (segment (start 119.786 74.786) (end 120 75) (width 0.2) (layer "F.Cu") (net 2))
 (via (at 101.714 72.1788) (size 0.6) (drill 0.3) (layers "F.Cu" "B.Cu") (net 1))
 (segment (start 101.714 87.714) (end 101.714 72.1788) (width 0.2) (layer "B.Cu") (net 1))
 (segment (start 107.46 93.46) (end 101.714 87.714) (width 0.2) (layer "B.Cu") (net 1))
 (segment (start 142.92 85.5) (end 138.92 81.5) (width 0.2) (layer "F.Cu") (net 12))
 (segment (start 137 81.5) (end 137 86.78) (width 0.2) (layer "F.Cu") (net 12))
 (segment (start 138.92 81.5) (end 137 81.5) (width 0.2) (layer "F.Cu") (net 12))
 (segment (start 137 86.78) (end 130.32 93.46) (width 0.2) (layer "F.Cu") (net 12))
 (segment (start 95.8835 72.1165) (end 104 64) (width 0.2) (layer "F.Cu") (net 3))
 (segment (start 91.5321 72.1165) (end 95.8835 72.1165) (width 0.2) (layer "F.Cu") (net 3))
 (via (at 104 64) (size 0.6) (drill 0.3) (layers "F.Cu" "B.Cu") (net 3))
 (via (at 117.5 64) (size 0.6) (drill 0.3) (layers "F.Cu" "B.Cu") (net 10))
 (segment (start 109.9212 71.5788) (end 117.5 64) (width 0.2) (layer "B.Cu") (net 10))
 (segment (start 91.5321 80.1165) (end 100.0698 71.5788) (width 0.2) (layer "B.Cu") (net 10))
 (segment (start 100.0698 71.5788) (end 109.9212 71.5788) (width 0.2) (layer "B.Cu") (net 10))
 (segment (start 127.5 57.5) (end 96 57.5) (width 0.2) (layer "F.Cu") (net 8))
 (segment (start 91.6921 61.8079) (end 91.6921 64.1165) (width 0.2) (layer "F.Cu") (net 8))
 (segment (start 96 57.5) (end 91.6921 61.8079) (width 0.2) (layer "F.Cu") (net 8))
 (segment (start 130.5 64) (end 130.5 60.5) (width 0.2) (layer "F.Cu") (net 8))
 (segment (start 130.5 60.5) (end 127.5 57.5) (width 0.2) (layer "F.Cu") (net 8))
 (segment (start 140.38 85.5) (end 137.94 87.94) (width 0.2) (layer "F.Cu") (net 13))
 (segment (start 137.94 87.94) (end 137.94 93.46) (width 0.2) (layer "F.Cu") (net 13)))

